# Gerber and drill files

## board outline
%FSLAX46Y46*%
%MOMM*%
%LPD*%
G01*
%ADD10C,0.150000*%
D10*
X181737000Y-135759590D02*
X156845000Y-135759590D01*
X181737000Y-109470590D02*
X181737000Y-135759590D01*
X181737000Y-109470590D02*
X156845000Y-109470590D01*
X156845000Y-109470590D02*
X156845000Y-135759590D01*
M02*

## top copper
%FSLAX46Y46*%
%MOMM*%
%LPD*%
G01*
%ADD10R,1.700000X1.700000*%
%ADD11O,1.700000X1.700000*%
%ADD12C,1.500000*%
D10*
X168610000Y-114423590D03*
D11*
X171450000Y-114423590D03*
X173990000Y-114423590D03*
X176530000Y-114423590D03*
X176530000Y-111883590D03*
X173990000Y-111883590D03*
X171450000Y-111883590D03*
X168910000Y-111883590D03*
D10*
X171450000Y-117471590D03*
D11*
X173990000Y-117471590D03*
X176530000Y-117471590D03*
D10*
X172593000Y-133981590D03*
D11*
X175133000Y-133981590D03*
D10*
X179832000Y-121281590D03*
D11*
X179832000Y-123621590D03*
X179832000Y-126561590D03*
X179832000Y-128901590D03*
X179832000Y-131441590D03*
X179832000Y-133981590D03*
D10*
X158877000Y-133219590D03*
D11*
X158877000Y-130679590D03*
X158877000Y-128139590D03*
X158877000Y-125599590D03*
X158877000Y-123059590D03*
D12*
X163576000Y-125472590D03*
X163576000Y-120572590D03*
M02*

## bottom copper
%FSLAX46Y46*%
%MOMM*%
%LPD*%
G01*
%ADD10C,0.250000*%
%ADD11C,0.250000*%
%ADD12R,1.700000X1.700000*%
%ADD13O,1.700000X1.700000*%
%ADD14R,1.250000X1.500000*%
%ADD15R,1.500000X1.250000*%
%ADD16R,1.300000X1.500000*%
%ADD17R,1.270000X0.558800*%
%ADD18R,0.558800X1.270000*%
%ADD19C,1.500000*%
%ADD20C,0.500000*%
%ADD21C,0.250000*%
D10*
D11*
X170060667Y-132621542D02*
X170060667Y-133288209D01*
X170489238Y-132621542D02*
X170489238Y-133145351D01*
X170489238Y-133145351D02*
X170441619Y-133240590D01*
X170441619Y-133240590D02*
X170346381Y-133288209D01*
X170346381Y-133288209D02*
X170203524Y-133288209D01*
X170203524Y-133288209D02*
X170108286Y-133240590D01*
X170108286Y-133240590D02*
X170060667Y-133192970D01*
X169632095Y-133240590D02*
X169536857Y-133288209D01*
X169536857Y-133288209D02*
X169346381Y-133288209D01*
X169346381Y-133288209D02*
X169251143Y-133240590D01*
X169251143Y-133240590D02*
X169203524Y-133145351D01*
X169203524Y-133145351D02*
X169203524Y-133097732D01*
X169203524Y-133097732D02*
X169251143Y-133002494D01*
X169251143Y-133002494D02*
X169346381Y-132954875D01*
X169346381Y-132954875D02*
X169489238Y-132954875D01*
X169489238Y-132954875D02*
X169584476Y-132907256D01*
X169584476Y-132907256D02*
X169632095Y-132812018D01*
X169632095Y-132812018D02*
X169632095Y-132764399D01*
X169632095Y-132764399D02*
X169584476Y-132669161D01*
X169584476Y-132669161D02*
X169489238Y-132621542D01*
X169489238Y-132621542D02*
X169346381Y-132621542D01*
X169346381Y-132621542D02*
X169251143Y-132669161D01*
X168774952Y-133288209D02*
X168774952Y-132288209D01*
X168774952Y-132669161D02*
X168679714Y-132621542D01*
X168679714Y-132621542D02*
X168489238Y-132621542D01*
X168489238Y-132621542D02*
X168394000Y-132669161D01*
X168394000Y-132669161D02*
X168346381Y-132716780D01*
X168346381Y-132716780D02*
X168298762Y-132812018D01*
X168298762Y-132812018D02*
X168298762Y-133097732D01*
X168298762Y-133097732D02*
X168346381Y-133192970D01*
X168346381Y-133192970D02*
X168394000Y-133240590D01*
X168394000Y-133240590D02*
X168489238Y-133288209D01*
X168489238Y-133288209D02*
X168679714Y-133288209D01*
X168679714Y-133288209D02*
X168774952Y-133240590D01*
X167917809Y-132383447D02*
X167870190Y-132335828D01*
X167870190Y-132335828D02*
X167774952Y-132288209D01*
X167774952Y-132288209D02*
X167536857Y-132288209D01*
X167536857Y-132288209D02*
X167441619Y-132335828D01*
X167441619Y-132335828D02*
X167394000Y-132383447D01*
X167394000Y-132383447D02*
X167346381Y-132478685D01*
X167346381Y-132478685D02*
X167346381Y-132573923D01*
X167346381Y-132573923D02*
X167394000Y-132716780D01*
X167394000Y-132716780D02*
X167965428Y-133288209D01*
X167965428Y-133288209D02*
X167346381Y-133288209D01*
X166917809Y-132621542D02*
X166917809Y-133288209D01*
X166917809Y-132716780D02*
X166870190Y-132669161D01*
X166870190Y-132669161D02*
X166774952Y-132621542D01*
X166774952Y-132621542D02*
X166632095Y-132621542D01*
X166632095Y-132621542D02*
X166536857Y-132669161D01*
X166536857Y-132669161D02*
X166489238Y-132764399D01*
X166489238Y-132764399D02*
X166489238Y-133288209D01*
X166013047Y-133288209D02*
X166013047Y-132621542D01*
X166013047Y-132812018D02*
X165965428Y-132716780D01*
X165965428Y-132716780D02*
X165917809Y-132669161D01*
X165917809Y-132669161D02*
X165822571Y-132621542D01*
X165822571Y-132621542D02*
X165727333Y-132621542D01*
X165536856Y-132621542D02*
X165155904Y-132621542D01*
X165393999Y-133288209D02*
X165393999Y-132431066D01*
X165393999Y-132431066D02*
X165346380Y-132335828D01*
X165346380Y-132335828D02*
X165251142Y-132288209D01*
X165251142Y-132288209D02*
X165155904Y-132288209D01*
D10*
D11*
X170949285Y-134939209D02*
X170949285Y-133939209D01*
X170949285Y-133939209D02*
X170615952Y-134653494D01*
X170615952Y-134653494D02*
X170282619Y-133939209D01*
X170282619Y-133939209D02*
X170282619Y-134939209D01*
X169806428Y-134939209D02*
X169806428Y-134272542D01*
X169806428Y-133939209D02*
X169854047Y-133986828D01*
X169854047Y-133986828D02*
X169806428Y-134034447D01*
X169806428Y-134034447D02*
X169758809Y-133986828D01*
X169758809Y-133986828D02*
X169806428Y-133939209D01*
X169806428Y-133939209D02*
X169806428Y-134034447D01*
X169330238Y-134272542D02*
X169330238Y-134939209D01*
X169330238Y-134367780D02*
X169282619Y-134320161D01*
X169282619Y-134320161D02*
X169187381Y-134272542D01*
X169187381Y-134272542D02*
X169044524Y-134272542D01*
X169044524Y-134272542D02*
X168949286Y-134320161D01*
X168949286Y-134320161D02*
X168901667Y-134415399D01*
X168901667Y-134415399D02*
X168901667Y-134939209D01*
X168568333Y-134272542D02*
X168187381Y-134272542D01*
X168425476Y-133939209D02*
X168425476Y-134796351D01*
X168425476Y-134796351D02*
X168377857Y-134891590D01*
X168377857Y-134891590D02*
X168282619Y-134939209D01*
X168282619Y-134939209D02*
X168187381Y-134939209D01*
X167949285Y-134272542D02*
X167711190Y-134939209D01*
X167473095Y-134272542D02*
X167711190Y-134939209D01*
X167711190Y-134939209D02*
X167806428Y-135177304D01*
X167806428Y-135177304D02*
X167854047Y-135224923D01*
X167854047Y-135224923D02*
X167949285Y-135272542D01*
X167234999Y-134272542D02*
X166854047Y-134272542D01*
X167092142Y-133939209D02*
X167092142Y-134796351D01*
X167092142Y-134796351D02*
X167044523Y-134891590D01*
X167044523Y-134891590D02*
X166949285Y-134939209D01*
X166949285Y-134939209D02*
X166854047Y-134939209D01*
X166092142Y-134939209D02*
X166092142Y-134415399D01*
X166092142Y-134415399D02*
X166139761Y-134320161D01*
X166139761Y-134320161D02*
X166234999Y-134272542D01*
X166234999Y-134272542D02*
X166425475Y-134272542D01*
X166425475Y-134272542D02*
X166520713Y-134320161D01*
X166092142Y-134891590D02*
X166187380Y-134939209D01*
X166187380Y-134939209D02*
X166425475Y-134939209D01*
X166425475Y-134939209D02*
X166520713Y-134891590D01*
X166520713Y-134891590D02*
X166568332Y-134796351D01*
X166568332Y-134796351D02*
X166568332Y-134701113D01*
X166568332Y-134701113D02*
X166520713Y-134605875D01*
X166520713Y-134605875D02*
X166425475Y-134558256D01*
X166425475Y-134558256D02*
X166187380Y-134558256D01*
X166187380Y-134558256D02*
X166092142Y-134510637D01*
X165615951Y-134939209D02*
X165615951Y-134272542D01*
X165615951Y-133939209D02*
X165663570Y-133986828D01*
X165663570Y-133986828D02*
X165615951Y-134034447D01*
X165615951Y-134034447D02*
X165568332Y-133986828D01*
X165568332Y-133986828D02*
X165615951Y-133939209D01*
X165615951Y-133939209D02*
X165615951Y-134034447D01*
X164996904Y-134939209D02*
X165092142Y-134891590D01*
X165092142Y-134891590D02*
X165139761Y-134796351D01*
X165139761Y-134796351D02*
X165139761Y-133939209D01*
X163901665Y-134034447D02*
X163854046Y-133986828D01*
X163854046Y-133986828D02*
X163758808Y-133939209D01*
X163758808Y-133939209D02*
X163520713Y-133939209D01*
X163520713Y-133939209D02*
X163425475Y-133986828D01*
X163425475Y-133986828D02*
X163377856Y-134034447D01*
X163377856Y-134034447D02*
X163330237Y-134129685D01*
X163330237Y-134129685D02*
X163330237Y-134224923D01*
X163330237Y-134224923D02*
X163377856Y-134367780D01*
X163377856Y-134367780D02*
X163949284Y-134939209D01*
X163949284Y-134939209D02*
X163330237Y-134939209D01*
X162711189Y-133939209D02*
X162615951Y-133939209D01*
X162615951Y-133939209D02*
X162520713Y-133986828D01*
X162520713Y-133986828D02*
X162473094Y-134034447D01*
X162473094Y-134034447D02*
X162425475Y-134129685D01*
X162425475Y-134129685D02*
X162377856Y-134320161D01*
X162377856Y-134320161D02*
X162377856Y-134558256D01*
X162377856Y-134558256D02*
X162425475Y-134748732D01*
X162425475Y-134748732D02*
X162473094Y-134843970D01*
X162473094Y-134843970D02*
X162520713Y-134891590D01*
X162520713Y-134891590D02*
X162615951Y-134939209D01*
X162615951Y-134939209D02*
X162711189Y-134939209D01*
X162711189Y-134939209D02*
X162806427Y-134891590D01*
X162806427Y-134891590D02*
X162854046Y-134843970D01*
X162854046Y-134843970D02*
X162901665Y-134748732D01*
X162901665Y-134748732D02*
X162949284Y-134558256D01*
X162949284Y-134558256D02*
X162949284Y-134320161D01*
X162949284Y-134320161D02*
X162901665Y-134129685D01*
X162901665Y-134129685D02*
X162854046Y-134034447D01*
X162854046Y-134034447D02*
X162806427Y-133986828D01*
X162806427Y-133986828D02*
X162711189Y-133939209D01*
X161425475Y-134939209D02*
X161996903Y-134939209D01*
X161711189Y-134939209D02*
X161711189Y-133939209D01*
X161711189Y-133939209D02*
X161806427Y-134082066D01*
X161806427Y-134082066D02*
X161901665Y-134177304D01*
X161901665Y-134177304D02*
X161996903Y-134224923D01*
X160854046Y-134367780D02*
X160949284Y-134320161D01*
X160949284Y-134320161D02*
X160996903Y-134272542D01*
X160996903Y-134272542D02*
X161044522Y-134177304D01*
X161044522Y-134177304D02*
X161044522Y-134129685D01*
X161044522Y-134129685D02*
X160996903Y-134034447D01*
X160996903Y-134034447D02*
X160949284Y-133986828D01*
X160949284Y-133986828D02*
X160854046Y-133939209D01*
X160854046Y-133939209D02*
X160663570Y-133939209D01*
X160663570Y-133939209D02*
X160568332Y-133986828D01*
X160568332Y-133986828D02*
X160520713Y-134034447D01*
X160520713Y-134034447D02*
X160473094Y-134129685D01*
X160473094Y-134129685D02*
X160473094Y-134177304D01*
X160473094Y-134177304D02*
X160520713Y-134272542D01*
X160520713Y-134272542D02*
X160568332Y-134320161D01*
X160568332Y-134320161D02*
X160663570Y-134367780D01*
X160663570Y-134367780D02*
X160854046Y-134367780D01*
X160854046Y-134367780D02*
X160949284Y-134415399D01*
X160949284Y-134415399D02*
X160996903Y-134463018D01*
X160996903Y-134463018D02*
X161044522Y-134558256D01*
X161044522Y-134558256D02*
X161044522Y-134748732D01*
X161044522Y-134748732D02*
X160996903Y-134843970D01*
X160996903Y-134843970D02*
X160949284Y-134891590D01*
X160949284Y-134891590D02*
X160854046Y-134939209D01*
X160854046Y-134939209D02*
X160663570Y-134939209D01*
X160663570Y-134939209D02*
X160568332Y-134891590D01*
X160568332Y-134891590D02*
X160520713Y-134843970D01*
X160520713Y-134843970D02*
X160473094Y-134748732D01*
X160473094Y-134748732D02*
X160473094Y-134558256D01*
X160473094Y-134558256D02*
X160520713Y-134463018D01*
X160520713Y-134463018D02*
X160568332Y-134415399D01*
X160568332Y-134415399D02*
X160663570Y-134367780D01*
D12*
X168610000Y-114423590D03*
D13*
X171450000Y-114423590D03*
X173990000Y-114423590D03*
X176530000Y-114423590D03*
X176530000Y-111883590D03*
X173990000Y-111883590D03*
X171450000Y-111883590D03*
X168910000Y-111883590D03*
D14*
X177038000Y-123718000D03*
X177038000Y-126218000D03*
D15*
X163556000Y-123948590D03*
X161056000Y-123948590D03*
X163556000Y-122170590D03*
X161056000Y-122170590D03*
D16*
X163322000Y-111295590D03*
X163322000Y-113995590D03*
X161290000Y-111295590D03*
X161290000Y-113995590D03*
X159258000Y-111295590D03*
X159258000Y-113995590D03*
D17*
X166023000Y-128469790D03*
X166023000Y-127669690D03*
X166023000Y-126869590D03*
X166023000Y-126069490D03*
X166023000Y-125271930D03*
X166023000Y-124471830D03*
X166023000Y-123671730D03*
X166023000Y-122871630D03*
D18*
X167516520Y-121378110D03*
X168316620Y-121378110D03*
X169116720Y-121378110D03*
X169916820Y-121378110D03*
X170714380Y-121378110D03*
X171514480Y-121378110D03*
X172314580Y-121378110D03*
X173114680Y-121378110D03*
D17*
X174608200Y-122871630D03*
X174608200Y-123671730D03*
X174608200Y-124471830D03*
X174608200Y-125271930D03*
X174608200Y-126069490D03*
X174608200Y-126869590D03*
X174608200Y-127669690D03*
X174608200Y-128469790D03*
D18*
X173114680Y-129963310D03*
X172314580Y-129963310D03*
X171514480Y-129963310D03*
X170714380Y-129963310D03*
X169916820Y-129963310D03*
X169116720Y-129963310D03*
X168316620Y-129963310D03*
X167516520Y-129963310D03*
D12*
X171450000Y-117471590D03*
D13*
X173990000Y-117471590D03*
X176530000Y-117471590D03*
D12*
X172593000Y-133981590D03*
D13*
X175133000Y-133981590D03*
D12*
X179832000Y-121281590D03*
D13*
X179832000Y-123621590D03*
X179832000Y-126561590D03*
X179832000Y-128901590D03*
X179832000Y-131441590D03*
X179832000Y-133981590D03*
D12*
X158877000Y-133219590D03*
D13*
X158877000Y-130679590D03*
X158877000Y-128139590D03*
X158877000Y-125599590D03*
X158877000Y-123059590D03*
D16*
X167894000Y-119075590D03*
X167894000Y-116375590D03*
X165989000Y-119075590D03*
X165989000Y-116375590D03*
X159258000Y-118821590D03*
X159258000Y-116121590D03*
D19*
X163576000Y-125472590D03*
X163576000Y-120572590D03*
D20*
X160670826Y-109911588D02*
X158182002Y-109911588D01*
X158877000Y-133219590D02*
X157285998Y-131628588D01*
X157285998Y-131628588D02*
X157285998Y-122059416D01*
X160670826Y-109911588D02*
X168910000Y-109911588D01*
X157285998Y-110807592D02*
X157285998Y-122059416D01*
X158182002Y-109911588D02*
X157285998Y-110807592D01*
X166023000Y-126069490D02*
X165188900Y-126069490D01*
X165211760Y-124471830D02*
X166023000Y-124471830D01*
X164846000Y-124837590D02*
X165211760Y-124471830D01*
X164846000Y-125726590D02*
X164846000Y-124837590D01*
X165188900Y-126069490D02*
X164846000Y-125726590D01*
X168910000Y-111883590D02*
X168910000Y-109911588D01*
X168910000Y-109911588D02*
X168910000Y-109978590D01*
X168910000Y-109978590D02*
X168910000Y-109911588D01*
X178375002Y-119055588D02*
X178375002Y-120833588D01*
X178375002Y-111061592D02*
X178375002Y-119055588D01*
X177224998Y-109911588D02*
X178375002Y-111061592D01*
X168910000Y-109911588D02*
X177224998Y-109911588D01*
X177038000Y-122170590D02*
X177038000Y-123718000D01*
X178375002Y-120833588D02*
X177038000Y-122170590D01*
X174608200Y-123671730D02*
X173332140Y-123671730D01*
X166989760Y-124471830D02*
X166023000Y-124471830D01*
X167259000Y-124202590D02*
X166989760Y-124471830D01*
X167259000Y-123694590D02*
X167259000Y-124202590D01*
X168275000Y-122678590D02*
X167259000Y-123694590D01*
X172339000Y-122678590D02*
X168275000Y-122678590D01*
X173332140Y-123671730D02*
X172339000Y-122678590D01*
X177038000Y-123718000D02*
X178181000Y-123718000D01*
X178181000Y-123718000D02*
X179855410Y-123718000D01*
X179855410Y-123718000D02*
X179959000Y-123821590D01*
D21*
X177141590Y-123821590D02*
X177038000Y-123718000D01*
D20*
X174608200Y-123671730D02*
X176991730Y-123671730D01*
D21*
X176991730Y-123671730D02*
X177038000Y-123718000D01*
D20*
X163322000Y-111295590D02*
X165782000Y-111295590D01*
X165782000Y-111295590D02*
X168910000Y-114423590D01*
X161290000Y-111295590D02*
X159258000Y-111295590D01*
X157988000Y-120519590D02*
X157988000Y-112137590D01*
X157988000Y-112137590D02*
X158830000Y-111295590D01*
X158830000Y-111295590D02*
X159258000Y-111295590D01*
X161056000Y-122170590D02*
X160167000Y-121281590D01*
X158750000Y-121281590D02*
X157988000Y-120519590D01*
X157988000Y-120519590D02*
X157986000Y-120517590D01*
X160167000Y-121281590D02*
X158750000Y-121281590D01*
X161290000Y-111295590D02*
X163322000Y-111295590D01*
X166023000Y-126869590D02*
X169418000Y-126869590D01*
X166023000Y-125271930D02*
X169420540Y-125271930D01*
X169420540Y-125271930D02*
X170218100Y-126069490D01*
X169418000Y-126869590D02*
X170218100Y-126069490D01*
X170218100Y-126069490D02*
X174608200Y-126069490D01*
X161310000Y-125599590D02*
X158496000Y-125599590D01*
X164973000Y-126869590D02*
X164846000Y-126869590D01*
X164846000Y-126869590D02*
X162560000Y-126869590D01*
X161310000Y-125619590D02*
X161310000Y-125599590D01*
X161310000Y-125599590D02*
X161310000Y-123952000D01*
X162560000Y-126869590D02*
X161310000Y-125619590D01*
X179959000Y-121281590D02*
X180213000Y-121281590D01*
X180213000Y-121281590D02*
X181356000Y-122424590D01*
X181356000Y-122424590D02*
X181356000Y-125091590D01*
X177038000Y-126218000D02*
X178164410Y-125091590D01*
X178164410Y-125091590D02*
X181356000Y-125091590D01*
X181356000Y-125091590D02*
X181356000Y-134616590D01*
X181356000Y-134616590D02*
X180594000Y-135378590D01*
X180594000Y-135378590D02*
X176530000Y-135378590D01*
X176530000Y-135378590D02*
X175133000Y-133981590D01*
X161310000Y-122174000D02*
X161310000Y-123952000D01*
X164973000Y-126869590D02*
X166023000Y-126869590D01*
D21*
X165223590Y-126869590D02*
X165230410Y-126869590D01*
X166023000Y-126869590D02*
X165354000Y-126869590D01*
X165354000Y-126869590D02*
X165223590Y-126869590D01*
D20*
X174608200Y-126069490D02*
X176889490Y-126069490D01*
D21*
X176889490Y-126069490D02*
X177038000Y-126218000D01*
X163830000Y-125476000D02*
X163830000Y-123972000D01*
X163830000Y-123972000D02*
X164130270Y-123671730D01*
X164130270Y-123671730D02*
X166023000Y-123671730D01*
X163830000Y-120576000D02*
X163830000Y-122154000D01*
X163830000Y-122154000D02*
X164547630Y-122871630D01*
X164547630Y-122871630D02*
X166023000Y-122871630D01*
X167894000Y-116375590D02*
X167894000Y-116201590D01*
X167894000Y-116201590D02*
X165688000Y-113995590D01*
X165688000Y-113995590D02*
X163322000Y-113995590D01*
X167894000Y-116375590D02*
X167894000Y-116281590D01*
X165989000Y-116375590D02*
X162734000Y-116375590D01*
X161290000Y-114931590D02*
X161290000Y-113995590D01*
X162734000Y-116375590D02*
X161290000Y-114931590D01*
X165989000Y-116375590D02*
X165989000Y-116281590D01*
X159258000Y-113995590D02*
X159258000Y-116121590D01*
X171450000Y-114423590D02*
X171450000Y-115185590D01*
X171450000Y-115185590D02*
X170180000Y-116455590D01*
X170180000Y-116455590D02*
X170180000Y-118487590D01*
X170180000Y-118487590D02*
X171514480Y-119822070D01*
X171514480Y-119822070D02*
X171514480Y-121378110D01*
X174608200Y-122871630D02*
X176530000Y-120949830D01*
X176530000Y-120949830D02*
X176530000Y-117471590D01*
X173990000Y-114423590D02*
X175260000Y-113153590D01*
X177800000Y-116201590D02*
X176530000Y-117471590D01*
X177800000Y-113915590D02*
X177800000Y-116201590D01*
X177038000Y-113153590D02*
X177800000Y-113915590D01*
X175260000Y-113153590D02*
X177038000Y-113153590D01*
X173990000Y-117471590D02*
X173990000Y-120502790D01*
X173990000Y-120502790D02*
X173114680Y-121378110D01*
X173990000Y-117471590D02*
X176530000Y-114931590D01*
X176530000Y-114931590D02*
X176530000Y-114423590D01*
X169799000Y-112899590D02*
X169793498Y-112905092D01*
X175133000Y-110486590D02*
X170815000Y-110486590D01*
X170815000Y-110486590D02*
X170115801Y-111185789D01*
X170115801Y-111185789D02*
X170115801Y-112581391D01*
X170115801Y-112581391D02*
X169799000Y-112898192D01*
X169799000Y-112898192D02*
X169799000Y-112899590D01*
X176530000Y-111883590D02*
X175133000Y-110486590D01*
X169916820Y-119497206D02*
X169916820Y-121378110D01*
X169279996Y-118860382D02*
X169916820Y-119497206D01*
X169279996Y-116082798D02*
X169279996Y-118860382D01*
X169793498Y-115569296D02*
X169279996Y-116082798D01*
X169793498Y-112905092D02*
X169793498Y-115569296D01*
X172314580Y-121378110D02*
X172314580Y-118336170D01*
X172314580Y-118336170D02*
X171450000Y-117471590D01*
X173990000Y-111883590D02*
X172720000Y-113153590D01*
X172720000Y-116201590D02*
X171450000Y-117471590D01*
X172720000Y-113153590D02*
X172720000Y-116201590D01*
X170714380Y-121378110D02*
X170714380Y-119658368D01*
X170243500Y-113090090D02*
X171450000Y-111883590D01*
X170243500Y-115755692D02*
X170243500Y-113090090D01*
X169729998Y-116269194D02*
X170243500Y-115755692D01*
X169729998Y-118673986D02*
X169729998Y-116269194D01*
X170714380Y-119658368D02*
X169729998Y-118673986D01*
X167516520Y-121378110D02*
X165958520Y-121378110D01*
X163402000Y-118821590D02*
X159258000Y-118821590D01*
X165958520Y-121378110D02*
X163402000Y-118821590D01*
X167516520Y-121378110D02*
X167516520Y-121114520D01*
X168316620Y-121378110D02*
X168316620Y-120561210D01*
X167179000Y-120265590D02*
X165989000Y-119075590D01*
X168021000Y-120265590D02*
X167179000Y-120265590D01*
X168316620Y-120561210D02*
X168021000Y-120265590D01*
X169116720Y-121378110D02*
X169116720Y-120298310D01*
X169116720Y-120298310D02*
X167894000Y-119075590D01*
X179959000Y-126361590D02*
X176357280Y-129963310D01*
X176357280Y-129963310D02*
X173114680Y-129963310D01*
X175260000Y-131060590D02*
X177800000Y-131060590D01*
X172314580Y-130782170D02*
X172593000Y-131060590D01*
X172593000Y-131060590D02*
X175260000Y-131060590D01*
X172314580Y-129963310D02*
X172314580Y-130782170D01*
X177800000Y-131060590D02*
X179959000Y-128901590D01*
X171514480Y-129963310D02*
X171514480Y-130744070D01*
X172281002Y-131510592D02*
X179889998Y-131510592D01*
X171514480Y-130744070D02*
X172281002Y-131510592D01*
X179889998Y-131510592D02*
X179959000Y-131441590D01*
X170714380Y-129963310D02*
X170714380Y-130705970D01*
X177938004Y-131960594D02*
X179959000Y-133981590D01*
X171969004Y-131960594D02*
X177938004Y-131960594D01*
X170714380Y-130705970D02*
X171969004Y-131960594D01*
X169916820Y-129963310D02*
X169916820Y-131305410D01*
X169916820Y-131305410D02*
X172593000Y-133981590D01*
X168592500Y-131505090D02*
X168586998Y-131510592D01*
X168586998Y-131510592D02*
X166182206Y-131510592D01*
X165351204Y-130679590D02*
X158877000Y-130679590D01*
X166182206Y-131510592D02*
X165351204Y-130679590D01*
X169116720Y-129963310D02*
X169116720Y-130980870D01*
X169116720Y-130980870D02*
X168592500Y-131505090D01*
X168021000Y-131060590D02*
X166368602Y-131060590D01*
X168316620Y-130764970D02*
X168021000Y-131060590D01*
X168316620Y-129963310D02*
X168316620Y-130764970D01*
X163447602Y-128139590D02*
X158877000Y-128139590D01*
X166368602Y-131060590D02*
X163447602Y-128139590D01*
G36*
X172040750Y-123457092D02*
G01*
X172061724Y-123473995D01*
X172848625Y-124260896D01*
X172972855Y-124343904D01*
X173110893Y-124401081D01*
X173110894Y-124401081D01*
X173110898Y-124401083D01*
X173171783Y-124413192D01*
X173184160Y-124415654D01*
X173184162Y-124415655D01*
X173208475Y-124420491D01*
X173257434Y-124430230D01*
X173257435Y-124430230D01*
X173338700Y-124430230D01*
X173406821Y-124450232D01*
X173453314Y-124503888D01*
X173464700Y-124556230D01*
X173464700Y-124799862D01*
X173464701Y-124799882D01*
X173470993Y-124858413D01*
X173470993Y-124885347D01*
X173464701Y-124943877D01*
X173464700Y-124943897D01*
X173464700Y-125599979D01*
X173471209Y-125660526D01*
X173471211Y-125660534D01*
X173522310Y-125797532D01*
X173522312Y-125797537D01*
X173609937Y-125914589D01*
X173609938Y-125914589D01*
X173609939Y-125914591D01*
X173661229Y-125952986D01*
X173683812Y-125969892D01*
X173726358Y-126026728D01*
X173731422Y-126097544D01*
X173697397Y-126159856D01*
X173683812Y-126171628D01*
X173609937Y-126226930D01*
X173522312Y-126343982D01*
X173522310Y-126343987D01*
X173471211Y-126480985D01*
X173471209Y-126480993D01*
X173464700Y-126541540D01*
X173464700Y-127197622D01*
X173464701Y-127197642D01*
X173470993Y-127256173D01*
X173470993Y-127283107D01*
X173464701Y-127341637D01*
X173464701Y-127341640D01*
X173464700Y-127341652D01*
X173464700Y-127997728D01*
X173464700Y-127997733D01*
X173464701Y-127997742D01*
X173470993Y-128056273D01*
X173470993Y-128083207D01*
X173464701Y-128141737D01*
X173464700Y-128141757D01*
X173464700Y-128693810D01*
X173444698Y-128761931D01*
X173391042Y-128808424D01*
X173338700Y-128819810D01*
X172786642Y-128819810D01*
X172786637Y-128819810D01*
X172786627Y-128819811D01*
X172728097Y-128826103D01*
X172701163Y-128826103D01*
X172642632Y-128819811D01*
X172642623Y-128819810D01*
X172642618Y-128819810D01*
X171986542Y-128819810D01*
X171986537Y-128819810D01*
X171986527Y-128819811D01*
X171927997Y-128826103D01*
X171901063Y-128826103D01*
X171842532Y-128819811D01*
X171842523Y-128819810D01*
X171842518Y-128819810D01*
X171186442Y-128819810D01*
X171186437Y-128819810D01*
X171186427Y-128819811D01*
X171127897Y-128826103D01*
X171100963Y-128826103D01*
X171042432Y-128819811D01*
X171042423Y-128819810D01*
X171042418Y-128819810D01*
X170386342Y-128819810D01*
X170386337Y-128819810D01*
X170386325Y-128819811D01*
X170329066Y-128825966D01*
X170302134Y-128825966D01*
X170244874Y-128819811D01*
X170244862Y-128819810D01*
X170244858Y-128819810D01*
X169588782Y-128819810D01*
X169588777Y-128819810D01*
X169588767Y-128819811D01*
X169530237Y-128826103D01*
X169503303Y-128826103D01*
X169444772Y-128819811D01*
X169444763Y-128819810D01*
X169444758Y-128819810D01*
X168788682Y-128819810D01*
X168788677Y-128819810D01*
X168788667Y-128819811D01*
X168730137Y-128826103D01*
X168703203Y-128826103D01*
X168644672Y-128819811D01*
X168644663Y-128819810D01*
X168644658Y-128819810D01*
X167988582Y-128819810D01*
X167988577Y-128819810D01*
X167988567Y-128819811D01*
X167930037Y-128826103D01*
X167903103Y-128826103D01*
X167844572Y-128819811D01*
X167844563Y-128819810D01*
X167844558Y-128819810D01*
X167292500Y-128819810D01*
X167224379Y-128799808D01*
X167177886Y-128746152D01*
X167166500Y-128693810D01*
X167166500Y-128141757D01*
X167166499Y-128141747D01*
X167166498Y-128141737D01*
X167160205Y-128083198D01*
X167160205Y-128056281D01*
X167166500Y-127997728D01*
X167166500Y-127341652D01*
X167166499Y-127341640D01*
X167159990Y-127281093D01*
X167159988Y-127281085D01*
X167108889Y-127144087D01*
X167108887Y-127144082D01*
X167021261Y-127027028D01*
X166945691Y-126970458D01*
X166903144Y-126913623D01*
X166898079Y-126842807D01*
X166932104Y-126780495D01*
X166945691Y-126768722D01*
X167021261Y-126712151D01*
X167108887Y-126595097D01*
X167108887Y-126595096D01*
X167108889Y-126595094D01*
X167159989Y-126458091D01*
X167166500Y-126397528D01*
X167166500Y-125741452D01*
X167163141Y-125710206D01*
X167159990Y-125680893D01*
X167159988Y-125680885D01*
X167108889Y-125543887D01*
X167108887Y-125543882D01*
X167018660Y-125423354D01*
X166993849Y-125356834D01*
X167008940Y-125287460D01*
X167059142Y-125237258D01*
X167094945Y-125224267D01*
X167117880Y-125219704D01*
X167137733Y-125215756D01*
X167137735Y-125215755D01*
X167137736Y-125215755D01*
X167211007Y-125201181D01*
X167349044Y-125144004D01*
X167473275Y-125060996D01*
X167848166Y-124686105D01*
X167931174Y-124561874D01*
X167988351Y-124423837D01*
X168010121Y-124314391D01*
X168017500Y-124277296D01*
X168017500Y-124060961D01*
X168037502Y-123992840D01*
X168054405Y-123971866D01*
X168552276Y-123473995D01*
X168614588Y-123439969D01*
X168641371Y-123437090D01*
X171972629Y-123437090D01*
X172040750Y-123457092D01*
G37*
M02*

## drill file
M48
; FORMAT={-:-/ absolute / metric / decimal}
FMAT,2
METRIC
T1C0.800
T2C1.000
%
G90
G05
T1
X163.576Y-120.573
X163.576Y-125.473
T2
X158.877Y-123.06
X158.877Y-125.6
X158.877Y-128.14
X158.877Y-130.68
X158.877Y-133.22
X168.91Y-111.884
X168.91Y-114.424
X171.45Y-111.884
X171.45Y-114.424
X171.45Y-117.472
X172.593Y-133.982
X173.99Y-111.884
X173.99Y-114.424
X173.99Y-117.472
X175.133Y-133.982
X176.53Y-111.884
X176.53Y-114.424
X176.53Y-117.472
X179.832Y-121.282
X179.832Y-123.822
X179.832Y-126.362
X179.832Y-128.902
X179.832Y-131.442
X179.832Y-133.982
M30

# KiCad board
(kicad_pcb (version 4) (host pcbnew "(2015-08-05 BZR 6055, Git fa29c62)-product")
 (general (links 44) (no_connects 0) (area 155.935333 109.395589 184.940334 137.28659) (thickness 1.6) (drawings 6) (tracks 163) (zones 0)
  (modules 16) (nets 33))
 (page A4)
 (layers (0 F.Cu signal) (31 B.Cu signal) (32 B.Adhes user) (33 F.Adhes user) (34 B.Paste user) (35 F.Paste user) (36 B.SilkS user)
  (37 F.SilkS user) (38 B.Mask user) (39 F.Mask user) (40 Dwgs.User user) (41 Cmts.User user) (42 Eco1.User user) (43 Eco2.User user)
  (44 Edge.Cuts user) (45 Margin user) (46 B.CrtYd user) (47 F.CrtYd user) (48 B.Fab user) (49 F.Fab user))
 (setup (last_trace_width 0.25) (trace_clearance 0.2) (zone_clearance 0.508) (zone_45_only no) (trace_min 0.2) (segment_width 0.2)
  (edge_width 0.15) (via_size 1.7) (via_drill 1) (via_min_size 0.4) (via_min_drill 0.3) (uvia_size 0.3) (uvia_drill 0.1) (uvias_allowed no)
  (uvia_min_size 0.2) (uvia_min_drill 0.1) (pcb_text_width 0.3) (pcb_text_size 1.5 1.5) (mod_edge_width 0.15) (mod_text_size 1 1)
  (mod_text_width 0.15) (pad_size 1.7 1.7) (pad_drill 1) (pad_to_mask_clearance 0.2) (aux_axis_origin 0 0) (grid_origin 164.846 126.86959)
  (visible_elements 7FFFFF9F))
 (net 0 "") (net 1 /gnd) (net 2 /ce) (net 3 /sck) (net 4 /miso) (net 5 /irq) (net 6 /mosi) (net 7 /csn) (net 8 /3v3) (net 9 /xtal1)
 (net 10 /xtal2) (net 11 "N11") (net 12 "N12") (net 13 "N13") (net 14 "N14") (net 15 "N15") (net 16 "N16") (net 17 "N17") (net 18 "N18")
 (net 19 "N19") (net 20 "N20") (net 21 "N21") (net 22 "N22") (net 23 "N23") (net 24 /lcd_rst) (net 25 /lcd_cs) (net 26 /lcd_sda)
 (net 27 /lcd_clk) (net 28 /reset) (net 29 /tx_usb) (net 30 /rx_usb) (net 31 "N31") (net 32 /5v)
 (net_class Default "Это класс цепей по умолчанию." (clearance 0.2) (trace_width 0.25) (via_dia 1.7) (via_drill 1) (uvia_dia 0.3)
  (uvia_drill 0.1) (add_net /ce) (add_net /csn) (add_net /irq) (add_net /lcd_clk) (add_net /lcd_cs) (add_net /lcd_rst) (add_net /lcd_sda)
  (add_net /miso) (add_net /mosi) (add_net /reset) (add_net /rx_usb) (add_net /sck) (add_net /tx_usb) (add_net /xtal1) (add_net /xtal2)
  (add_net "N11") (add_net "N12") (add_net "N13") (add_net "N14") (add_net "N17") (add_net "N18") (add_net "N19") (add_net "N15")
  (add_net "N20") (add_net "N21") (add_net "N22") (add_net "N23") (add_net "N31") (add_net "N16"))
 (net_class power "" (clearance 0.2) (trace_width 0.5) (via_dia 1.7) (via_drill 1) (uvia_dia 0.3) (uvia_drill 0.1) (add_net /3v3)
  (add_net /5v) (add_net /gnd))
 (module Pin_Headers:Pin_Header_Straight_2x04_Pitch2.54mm (layer F.Cu) (at 168.91 114.42359 90)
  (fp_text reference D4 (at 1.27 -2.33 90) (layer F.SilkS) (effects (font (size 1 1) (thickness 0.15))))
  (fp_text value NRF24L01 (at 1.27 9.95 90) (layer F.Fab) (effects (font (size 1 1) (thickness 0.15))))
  (pad 1 thru_hole rect (at 0 0 90) (size 1.7 1.7) (drill 1 (offset 0 -0.3)) (layers *.Cu *.Mask) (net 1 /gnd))
  (pad 2 thru_hole oval (at 0 2.54 90) (size 1.7 1.7) (drill 1) (layers *.Cu *.Mask) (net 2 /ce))
  (pad 3 thru_hole oval (at 0 5.08 90) (size 1.7 1.7) (drill 1) (layers *.Cu *.Mask) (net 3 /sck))
  (pad 4 thru_hole oval (at 0 7.62 90) (size 1.7 1.7) (drill 1) (layers *.Cu *.Mask) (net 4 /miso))
  (pad 5 thru_hole oval (at 2.54 7.62 90) (size 1.7 1.7) (drill 1) (layers *.Cu *.Mask) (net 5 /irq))
  (pad 6 thru_hole oval (at 2.54 5.08 90) (size 1.7 1.7) (drill 1) (layers *.Cu *.Mask) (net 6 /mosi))
  (pad 7 thru_hole oval (at 2.54 2.54 90) (size 1.7 1.7) (drill 1) (layers *.Cu *.Mask) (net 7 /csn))
  (pad 8 thru_hole oval (at 2.54 0 90) (size 1.7 1.7) (drill 1) (layers *.Cu *.Mask) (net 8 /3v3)))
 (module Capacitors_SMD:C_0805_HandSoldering (layer B.Cu) (at 177.038 124.968 270)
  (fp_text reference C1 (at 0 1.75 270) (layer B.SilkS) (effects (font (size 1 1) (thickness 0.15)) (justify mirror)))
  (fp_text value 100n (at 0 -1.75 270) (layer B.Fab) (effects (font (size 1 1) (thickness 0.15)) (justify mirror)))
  (pad 1 smd rect (at -1.25 0 270) (size 1.5 1.25) (layers B.Cu B.Paste B.Mask) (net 8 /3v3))
  (pad 2 smd rect (at 1.25 0 270) (size 1.5 1.25) (layers B.Cu B.Paste B.Mask) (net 1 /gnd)))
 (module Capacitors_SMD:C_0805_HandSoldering (layer B.Cu) (at 162.306 123.94859 180)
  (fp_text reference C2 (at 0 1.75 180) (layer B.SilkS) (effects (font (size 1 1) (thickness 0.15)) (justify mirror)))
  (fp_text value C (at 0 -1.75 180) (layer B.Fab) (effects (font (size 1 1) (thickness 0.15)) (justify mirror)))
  (pad 1 smd rect (at -1.25 0 180) (size 1.5 1.25) (layers B.Cu B.Paste B.Mask) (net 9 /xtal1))
  (pad 2 smd rect (at 1.25 0 180) (size 1.5 1.25) (layers B.Cu B.Paste B.Mask) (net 1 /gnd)))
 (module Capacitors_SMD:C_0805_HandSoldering (layer B.Cu) (at 162.306 122.17059 180)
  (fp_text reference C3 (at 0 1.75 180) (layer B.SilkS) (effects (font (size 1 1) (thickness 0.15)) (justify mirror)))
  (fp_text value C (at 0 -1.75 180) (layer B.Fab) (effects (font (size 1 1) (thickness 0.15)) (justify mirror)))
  (pad 1 smd rect (at -1.25 0 180) (size 1.5 1.25) (layers B.Cu B.Paste B.Mask) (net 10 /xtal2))
  (pad 2 smd rect (at 1.25 0 180) (size 1.5 1.25) (layers B.Cu B.Paste B.Mask) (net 1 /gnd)))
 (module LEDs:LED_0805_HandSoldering (layer B.Cu) (at 163.322 112.64559 270)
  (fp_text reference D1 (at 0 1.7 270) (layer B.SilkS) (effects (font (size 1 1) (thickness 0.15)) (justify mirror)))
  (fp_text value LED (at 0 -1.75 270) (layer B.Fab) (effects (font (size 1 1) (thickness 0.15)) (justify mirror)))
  (pad 1 smd rect (at -1.35 0 270) (size 1.5 1.3) (layers B.Cu B.Paste B.Mask) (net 1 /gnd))
  (pad 2 smd rect (at 1.35 0 270) (size 1.5 1.3) (layers B.Cu B.Paste B.Mask) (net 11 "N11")))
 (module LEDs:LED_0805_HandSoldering (layer B.Cu) (at 161.29 112.64559 270)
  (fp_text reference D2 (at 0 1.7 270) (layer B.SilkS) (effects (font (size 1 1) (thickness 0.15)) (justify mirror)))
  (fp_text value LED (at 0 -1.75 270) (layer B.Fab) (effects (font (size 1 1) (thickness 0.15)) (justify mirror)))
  (pad 1 smd rect (at -1.35 0 270) (size 1.5 1.3) (layers B.Cu B.Paste B.Mask) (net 1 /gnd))
  (pad 2 smd rect (at 1.35 0 270) (size 1.5 1.3) (layers B.Cu B.Paste B.Mask) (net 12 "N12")))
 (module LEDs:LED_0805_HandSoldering (layer B.Cu) (at 159.258 112.64559 270)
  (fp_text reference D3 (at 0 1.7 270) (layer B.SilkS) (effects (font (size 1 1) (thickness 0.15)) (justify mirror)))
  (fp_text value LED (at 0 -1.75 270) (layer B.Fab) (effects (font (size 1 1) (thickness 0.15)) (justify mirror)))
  (pad 1 smd rect (at -1.35 0 270) (size 1.5 1.3) (layers B.Cu B.Paste B.Mask) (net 1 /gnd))
  (pad 2 smd rect (at 1.35 0 270) (size 1.5 1.3) (layers B.Cu B.Paste B.Mask) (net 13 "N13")))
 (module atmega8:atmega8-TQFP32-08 (layer B.Cu) (at 170.3156 125.67071)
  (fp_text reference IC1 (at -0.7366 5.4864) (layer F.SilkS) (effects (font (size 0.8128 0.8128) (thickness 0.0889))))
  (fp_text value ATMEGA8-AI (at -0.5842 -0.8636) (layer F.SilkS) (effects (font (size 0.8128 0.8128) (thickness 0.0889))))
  (pad 1 smd rect (at -4.2926 2.79908) (size 1.27 0.5588) (layers B.Cu B.Paste B.Mask) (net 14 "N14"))
  (pad 2 smd rect (at -4.2926 1.99898) (size 1.27 0.5588) (layers B.Cu B.Paste B.Mask) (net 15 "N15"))
  (pad 3 smd rect (at -4.2926 1.19888) (size 1.27 0.5588) (layers B.Cu B.Paste B.Mask) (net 1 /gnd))
  (pad 4 smd rect (at -4.2926 0.39878) (size 1.27 0.5588) (layers B.Cu B.Paste B.Mask) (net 8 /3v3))
  (pad 5 smd rect (at -4.2926 -0.39878) (size 1.27 0.5588) (layers B.Cu B.Paste B.Mask) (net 1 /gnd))
  (pad 6 smd rect (at -4.2926 -1.19888) (size 1.27 0.5588) (layers B.Cu B.Paste B.Mask) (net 8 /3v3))
  (pad 7 smd rect (at -4.2926 -1.99898) (size 1.27 0.5588) (layers B.Cu B.Paste B.Mask) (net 9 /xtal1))
  (pad 8 smd rect (at -4.2926 -2.79908) (size 1.27 0.5588) (layers B.Cu B.Paste B.Mask) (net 10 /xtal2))
  (pad 9 smd rect (at -2.79908 -4.2926) (size 0.5588 1.27) (layers B.Cu B.Paste B.Mask) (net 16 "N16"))
  (pad 10 smd rect (at -1.99898 -4.2926) (size 0.5588 1.27) (layers B.Cu B.Paste B.Mask) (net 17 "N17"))
  (pad 11 smd rect (at -1.19888 -4.2926) (size 0.5588 1.27) (layers B.Cu B.Paste B.Mask) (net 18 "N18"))
  (pad 12 smd rect (at -0.39878 -4.2926) (size 0.5588 1.27) (layers B.Cu B.Paste B.Mask) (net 5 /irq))
  (pad 13 smd rect (at 0.39878 -4.2926) (size 0.5588 1.27) (layers B.Cu B.Paste B.Mask) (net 7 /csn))
  (pad 14 smd rect (at 1.19888 -4.2926) (size 0.5588 1.27) (layers B.Cu B.Paste B.Mask) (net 2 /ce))
  (pad 15 smd rect (at 1.99898 -4.2926) (size 0.5588 1.27) (layers B.Cu B.Paste B.Mask) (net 6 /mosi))
  (pad 16 smd rect (at 2.79908 -4.2926) (size 0.5588 1.27) (layers B.Cu B.Paste B.Mask) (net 4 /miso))
  (pad 17 smd rect (at 4.2926 -2.79908) (size 1.27 0.5588) (layers B.Cu B.Paste B.Mask) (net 3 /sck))
  (pad 18 smd rect (at 4.2926 -1.99898) (size 1.27 0.5588) (layers B.Cu B.Paste B.Mask) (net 8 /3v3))
  (pad 19 smd rect (at 4.2926 -1.19888) (size 1.27 0.5588) (layers B.Cu B.Paste B.Mask) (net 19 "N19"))
  (pad 20 smd rect (at 4.2926 -0.39878) (size 1.27 0.5588) (layers B.Cu B.Paste B.Mask) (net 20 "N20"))
  (pad 21 smd rect (at 4.2926 0.39878) (size 1.27 0.5588) (layers B.Cu B.Paste B.Mask) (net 1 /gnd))
  (pad 22 smd rect (at 4.2926 1.19888) (size 1.27 0.5588) (layers B.Cu B.Paste B.Mask) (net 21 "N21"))
  (pad 23 smd rect (at 4.2926 1.99898) (size 1.27 0.5588) (layers B.Cu B.Paste B.Mask) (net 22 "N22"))
  (pad 24 smd rect (at 4.2926 2.79908) (size 1.27 0.5588) (layers B.Cu B.Paste B.Mask) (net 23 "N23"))
  (pad 25 smd rect (at 2.79908 4.2926) (size 0.5588 1.27) (layers B.Cu B.Paste B.Mask) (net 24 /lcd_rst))
  (pad 26 smd rect (at 1.99898 4.2926) (size 0.5588 1.27) (layers B.Cu B.Paste B.Mask) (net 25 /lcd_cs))
  (pad 27 smd rect (at 1.19888 4.2926) (size 0.5588 1.27) (layers B.Cu B.Paste B.Mask) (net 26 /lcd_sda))
  (pad 28 smd rect (at 0.39878 4.2926) (size 0.5588 1.27) (layers B.Cu B.Paste B.Mask) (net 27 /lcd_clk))
  (pad 29 smd rect (at -0.39878 4.2926) (size 0.5588 1.27) (layers B.Cu B.Paste B.Mask) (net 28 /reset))
  (pad 30 smd rect (at -1.19888 4.2926) (size 0.5588 1.27) (layers B.Cu B.Paste B.Mask) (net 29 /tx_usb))
  (pad 31 smd rect (at -1.99898 4.2926) (size 0.5588 1.27) (layers B.Cu B.Paste B.Mask) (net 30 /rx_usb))
  (pad 32 smd rect (at -2.79908 4.2926) (size 0.5588 1.27) (layers B.Cu B.Paste B.Mask) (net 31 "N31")))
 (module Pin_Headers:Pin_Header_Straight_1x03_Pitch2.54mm (layer F.Cu) (at 171.45 117.47159 90)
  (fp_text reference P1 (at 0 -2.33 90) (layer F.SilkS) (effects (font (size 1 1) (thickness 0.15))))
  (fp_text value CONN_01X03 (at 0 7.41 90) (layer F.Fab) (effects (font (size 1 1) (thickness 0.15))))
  (pad 1 thru_hole rect (at 0 0 90) (size 1.7 1.7) (drill 1) (layers *.Cu *.Mask) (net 6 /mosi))
  (pad 2 thru_hole oval (at 0 2.54 90) (size 1.7 1.7) (drill 1) (layers *.Cu *.Mask) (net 4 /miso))
  (pad 3 thru_hole oval (at 0 5.08 90) (size 1.7 1.7) (drill 1) (layers *.Cu *.Mask) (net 3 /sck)))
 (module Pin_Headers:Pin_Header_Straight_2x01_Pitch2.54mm (layer F.Cu) (at 172.593 133.98159)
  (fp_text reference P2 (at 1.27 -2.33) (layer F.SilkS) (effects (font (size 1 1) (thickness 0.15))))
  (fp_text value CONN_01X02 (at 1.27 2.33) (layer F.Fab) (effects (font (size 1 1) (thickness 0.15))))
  (pad 1 thru_hole rect (at 0 0) (size 1.7 1.7) (drill 1) (layers *.Cu *.Mask) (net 28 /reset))
  (pad 2 thru_hole oval (at 2.54 0) (size 1.7 1.7) (drill 1) (layers *.Cu *.Mask) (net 1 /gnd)))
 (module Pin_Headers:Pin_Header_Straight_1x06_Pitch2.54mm (layer F.Cu) (at 179.832 121.28159)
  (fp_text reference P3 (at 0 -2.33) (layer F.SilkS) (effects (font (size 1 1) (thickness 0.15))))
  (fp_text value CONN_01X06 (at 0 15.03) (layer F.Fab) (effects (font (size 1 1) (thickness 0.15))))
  (pad 1 thru_hole rect (at 0 0) (size 1.7 1.7) (drill 1) (layers *.Cu *.Mask) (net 1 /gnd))
  (pad 2 thru_hole oval (at 0 2.54) (size 1.7 1.7) (drill 1 (offset 0 -0.2)) (layers *.Cu *.Mask) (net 8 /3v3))
  (pad 3 thru_hole oval (at 0 5.08) (size 1.7 1.7) (drill 1 (offset 0 0.2)) (layers *.Cu *.Mask) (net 24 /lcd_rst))
  (pad 4 thru_hole oval (at 0 7.62) (size 1.7 1.7) (drill 1) (layers *.Cu *.Mask) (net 25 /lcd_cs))
  (pad 5 thru_hole oval (at 0 10.16) (size 1.7 1.7) (drill 1) (layers *.Cu *.Mask) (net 26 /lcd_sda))
  (pad 6 thru_hole oval (at 0 12.7) (size 1.7 1.7) (drill 1) (layers *.Cu *.Mask) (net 27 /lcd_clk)))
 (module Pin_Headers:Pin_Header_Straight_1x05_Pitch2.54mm (layer F.Cu) (at 158.877 133.21959 180)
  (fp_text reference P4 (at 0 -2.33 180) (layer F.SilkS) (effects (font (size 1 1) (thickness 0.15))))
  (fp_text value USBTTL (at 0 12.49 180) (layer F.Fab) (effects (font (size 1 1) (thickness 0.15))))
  (pad 1 thru_hole rect (at 0 0 180) (size 1.7 1.7) (drill 1) (layers *.Cu *.Mask) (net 8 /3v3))
  (pad 2 thru_hole oval (at 0 2.54 180) (size 1.7 1.7) (drill 1) (layers *.Cu *.Mask) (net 29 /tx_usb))
  (pad 3 thru_hole oval (at 0 5.08 180) (size 1.7 1.7) (drill 1) (layers *.Cu *.Mask) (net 30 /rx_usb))
  (pad 4 thru_hole oval (at 0 7.62 180) (size 1.7 1.7) (drill 1) (layers *.Cu *.Mask) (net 1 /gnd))
  (pad 5 thru_hole oval (at 0 10.16 180) (size 1.7 1.7) (drill 1) (layers *.Cu *.Mask) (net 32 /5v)))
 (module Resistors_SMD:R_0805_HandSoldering (layer B.Cu) (at 167.894 117.72559 90)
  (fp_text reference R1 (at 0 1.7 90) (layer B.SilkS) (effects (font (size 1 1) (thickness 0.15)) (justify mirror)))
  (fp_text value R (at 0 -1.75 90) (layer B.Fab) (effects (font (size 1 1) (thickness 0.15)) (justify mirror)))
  (pad 1 smd rect (at -1.35 0 90) (size 1.5 1.3) (layers B.Cu B.Paste B.Mask) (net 18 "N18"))
  (pad 2 smd rect (at 1.35 0 90) (size 1.5 1.3) (layers B.Cu B.Paste B.Mask) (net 11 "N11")))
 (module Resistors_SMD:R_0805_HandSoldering (layer B.Cu) (at 165.989 117.72559 90)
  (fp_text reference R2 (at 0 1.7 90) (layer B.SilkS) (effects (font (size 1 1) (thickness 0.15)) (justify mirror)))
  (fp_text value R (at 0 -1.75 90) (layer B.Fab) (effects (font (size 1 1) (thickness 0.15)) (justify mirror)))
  (pad 1 smd rect (at -1.35 0 90) (size 1.5 1.3) (layers B.Cu B.Paste B.Mask) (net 17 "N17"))
  (pad 2 smd rect (at 1.35 0 90) (size 1.5 1.3) (layers B.Cu B.Paste B.Mask) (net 12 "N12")))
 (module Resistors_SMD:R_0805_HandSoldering (layer B.Cu) (at 159.258 117.47159 90)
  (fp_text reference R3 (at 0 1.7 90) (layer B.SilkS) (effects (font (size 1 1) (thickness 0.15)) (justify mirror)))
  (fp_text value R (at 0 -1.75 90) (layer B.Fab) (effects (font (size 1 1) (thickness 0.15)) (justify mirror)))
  (pad 1 smd rect (at -1.35 0 90) (size 1.5 1.3) (layers B.Cu B.Paste B.Mask) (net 16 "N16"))
  (pad 2 smd rect (at 1.35 0 90) (size 1.5 1.3) (layers B.Cu B.Paste B.Mask) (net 13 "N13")))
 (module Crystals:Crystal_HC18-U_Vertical (layer F.Cu) (at 163.576 125.47259 90)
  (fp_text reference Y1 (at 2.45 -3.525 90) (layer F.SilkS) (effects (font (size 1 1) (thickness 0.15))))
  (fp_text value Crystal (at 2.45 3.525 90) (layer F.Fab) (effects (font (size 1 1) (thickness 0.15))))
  (pad 1 thru_hole circle (at 0 0 90) (size 1.5 1.5) (drill 0.8) (layers *.Cu *.Mask) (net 9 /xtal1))
  (pad 2 thru_hole circle (at 4.9 0 90) (size 1.5 1.5) (drill 0.8) (layers *.Cu *.Mask) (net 10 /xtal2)))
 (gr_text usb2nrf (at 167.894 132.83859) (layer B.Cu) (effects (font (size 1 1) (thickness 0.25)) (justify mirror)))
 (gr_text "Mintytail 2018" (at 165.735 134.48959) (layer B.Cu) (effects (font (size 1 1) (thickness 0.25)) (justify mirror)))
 (gr_line (start 181.737 135.75959) (end 156.845 135.75959) (angle 90) (layer Edge.Cuts) (width 0.15))
 (gr_line (start 181.737 109.47059) (end 181.737 135.75959) (angle 90) (layer Edge.Cuts) (width 0.15))
 (gr_line (start 181.737 109.47059) (end 156.845 109.47059) (angle 90) (layer Edge.Cuts) (width 0.15))
 (gr_line (start 156.845 109.47059) (end 156.845 135.75959) (angle 90) (layer Edge.Cuts) (width 0.15))
 (segment (start 160.670826 109.911588) (end 158.182002 109.911588) (width 0.5) (layer B.Cu) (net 8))
 (segment (start 158.877 133.21959) (end 157.285998 131.628588) (width 0.5) (layer B.Cu) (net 8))
 (segment (start 157.285998 131.628588) (end 157.285998 122.059416) (width 0.5) (layer B.Cu) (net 8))
 (segment (start 160.670826 109.911588) (end 168.91 109.911588) (width 0.5) (layer B.Cu) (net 8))
 (segment (start 157.285998 110.807592) (end 157.285998 122.059416) (width 0.5) (layer B.Cu) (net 8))
 (segment (start 158.182002 109.911588) (end 157.285998 110.807592) (width 0.5) (layer B.Cu) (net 8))
 (segment (start 166.023 126.06949) (end 165.1889 126.06949) (width 0.5) (layer B.Cu) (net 8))
 (segment (start 165.21176 124.47183) (end 166.023 124.47183) (width 0.5) (layer B.Cu) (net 8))
 (segment (start 164.846 124.83759) (end 165.21176 124.47183) (width 0.5) (layer B.Cu) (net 8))
 (segment (start 164.846 125.72659) (end 164.846 124.83759) (width 0.5) (layer B.Cu) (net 8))
 (segment (start 165.1889 126.06949) (end 164.846 125.72659) (width 0.5) (layer B.Cu) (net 8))
 (segment (start 168.91 111.88359) (end 168.91 109.911588) (width 0.5) (layer B.Cu) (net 8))
 (segment (start 168.91 109.911588) (end 168.91 109.97859) (width 0.5) (layer B.Cu) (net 8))
 (segment (start 168.91 109.97859) (end 168.91 109.911588) (width 0.5) (layer B.Cu) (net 8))
 (segment (start 178.375002 119.055588) (end 178.375002 120.833588) (width 0.5) (layer B.Cu) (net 8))
 (segment (start 178.375002 111.061592) (end 178.375002 119.055588) (width 0.5) (layer B.Cu) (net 8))
 (segment (start 177.224998 109.911588) (end 178.375002 111.061592) (width 0.5) (layer B.Cu) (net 8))
 (segment (start 168.91 109.911588) (end 177.224998 109.911588) (width 0.5) (layer B.Cu) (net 8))
 (segment (start 177.038 122.17059) (end 177.038 123.718) (width 0.5) (layer B.Cu) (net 8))
 (segment (start 178.375002 120.833588) (end 177.038 122.17059) (width 0.5) (layer B.Cu) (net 8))
 (segment (start 174.6082 123.67173) (end 173.33214 123.67173) (width 0.5) (layer B.Cu) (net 8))
 (segment (start 166.98976 124.47183) (end 166.023 124.47183) (width 0.5) (layer B.Cu) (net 8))
 (segment (start 167.259 124.20259) (end 166.98976 124.47183) (width 0.5) (layer B.Cu) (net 8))
 (segment (start 167.259 123.69459) (end 167.259 124.20259) (width 0.5) (layer B.Cu) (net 8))
 (segment (start 168.275 122.67859) (end 167.259 123.69459) (width 0.5) (layer B.Cu) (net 8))
 (segment (start 172.339 122.67859) (end 168.275 122.67859) (width 0.5) (layer B.Cu) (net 8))
 (segment (start 173.33214 123.67173) (end 172.339 122.67859) (width 0.5) (layer B.Cu) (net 8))
 (segment (start 177.038 123.718) (end 178.181 123.718) (width 0.5) (layer B.Cu) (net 8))
 (segment (start 178.181 123.718) (end 179.85541 123.718) (width 0.5) (layer B.Cu) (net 8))
 (segment (start 179.85541 123.718) (end 179.959 123.82159) (width 0.5) (layer B.Cu) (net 8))
 (segment (start 177.14159 123.82159) (end 177.038 123.718) (width 0.25) (layer B.Cu) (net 8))
 (segment (start 174.6082 123.67173) (end 176.99173 123.67173) (width 0.5) (layer B.Cu) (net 8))
 (segment (start 176.99173 123.67173) (end 177.038 123.718) (width 0.25) (layer B.Cu) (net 8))
 (segment (start 163.322 111.29559) (end 165.782 111.29559) (width 0.5) (layer B.Cu) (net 1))
 (segment (start 165.782 111.29559) (end 168.91 114.42359) (width 0.5) (layer B.Cu) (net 1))
 (segment (start 161.29 111.29559) (end 159.258 111.29559) (width 0.5) (layer B.Cu) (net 1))
 (segment (start 157.988 120.51959) (end 157.988 112.13759) (width 0.5) (layer B.Cu) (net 1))
 (segment (start 157.988 112.13759) (end 158.83 111.29559) (width 0.5) (layer B.Cu) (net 1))
 (segment (start 158.83 111.29559) (end 159.258 111.29559) (width 0.5) (layer B.Cu) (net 1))
 (segment (start 161.056 122.17059) (end 160.167 121.28159) (width 0.5) (layer B.Cu) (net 1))
 (segment (start 158.75 121.28159) (end 157.988 120.51959) (width 0.5) (layer B.Cu) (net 1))
 (segment (start 157.988 120.51959) (end 157.986 120.51759) (width 0.5) (layer B.Cu) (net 1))
 (segment (start 160.167 121.28159) (end 158.75 121.28159) (width 0.5) (layer B.Cu) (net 1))
 (segment (start 161.29 111.29559) (end 163.322 111.29559) (width 0.5) (layer B.Cu) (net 1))
 (segment (start 166.023 126.86959) (end 169.418 126.86959) (width 0.5) (layer B.Cu) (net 1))
 (segment (start 166.023 125.27193) (end 169.42054 125.27193) (width 0.5) (layer B.Cu) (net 1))
 (segment (start 169.42054 125.27193) (end 170.2181 126.06949) (width 0.5) (layer B.Cu) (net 1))
 (segment (start 169.418 126.86959) (end 170.2181 126.06949) (width 0.5) (layer B.Cu) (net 1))
 (segment (start 170.2181 126.06949) (end 174.6082 126.06949) (width 0.5) (layer B.Cu) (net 1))
 (segment (start 161.31 125.59959) (end 158.496 125.59959) (width 0.5) (layer B.Cu) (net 1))
 (segment (start 164.973 126.86959) (end 164.846 126.86959) (width 0.5) (layer B.Cu) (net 1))
 (segment (start 164.846 126.86959) (end 162.56 126.86959) (width 0.5) (layer B.Cu) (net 1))
 (segment (start 161.31 125.61959) (end 161.31 125.59959) (width 0.5) (layer B.Cu) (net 1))
 (segment (start 161.31 125.59959) (end 161.31 123.952) (width 0.5) (layer B.Cu) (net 1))
 (segment (start 162.56 126.86959) (end 161.31 125.61959) (width 0.5) (layer B.Cu) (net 1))
 (segment (start 179.959 121.28159) (end 180.213 121.28159) (width 0.5) (layer B.Cu) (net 1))
 (segment (start 180.213 121.28159) (end 181.356 122.42459) (width 0.5) (layer B.Cu) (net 1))
 (segment (start 181.356 122.42459) (end 181.356 125.09159) (width 0.5) (layer B.Cu) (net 1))
 (segment (start 177.038 126.218) (end 178.16441 125.09159) (width 0.5) (layer B.Cu) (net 1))
 (segment (start 178.16441 125.09159) (end 181.356 125.09159) (width 0.5) (layer B.Cu) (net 1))
 (segment (start 181.356 125.09159) (end 181.356 134.61659) (width 0.5) (layer B.Cu) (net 1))
 (segment (start 181.356 134.61659) (end 180.594 135.37859) (width 0.5) (layer B.Cu) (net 1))
 (segment (start 180.594 135.37859) (end 176.53 135.37859) (width 0.5) (layer B.Cu) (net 1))
 (segment (start 176.53 135.37859) (end 175.133 133.98159) (width 0.5) (layer B.Cu) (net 1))
 (segment (start 161.31 122.174) (end 161.31 123.952) (width 0.5) (layer B.Cu) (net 1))
 (segment (start 164.973 126.86959) (end 166.023 126.86959) (width 0.5) (layer B.Cu) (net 1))
 (segment (start 165.22359 126.86959) (end 165.23041 126.86959) (width 0.25) (layer B.Cu) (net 1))
 (segment (start 166.023 126.86959) (end 165.354 126.86959) (width 0.25) (layer B.Cu) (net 1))
 (segment (start 165.354 126.86959) (end 165.22359 126.86959) (width 0.25) (layer B.Cu) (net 1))
 (segment (start 174.6082 126.06949) (end 176.88949 126.06949) (width 0.5) (layer B.Cu) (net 1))
 (segment (start 176.88949 126.06949) (end 177.038 126.218) (width 0.25) (layer B.Cu) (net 1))
 (segment (start 163.83 125.476) (end 163.83 123.972) (width 0.25) (layer B.Cu) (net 9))
 (segment (start 163.83 123.972) (end 164.13027 123.67173) (width 0.25) (layer B.Cu) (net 9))
 (segment (start 164.13027 123.67173) (end 166.023 123.67173) (width 0.25) (layer B.Cu) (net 9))
 (segment (start 163.83 120.576) (end 163.83 122.154) (width 0.25) (layer B.Cu) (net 10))
 (segment (start 163.83 122.154) (end 164.54763 122.87163) (width 0.25) (layer B.Cu) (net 10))
 (segment (start 164.54763 122.87163) (end 166.023 122.87163) (width 0.25) (layer B.Cu) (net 10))
 (segment (start 167.894 116.37559) (end 167.894 116.20159) (width 0.25) (layer B.Cu) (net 11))
 (segment (start 167.894 116.20159) (end 165.688 113.99559) (width 0.25) (layer B.Cu) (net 11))
 (segment (start 165.688 113.99559) (end 163.322 113.99559) (width 0.25) (layer B.Cu) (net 11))
 (segment (start 167.894 116.37559) (end 167.894 116.28159) (width 0.25) (layer B.Cu) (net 11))
 (segment (start 165.989 116.37559) (end 162.734 116.37559) (width 0.25) (layer B.Cu) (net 12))
 (segment (start 161.29 114.93159) (end 161.29 113.99559) (width 0.25) (layer B.Cu) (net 12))
 (segment (start 162.734 116.37559) (end 161.29 114.93159) (width 0.25) (layer B.Cu) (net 12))
 (segment (start 165.989 116.37559) (end 165.989 116.28159) (width 0.25) (layer B.Cu) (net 12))
 (segment (start 159.258 113.99559) (end 159.258 116.12159) (width 0.25) (layer B.Cu) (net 13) (status C00000))
 (segment (start 171.45 114.42359) (end 171.45 115.18559) (width 0.25) (layer B.Cu) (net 2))
 (segment (start 171.45 115.18559) (end 170.18 116.45559) (width 0.25) (layer B.Cu) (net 2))
 (segment (start 170.18 116.45559) (end 170.18 118.48759) (width 0.25) (layer B.Cu) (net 2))
 (segment (start 170.18 118.48759) (end 171.51448 119.82207) (width 0.25) (layer B.Cu) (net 2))
 (segment (start 171.51448 119.82207) (end 171.51448 121.37811) (width 0.25) (layer B.Cu) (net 2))
 (segment (start 174.6082 122.87163) (end 176.53 120.94983) (width 0.25) (layer B.Cu) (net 3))
 (segment (start 176.53 120.94983) (end 176.53 117.47159) (width 0.25) (layer B.Cu) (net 3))
 (segment (start 173.99 114.42359) (end 175.26 113.15359) (width 0.25) (layer B.Cu) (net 3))
 (segment (start 177.8 116.20159) (end 176.53 117.47159) (width 0.25) (layer B.Cu) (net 3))
 (segment (start 177.8 113.91559) (end 177.8 116.20159) (width 0.25) (layer B.Cu) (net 3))
 (segment (start 177.038 113.15359) (end 177.8 113.91559) (width 0.25) (layer B.Cu) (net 3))
 (segment (start 175.26 113.15359) (end 177.038 113.15359) (width 0.25) (layer B.Cu) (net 3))
 (segment (start 173.99 117.47159) (end 173.99 120.50279) (width 0.25) (layer B.Cu) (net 4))
 (segment (start 173.99 120.50279) (end 173.11468 121.37811) (width 0.25) (layer B.Cu) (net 4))
 (segment (start 173.99 117.47159) (end 176.53 114.93159) (width 0.25) (layer B.Cu) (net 4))
 (segment (start 176.53 114.93159) (end 176.53 114.42359) (width 0.25) (layer B.Cu) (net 4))
 (segment (start 169.799 112.89959) (end 169.793498 112.905092) (width 0.25) (layer B.Cu) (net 5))
 (segment (start 175.133 110.48659) (end 170.815 110.48659) (width 0.25) (layer B.Cu) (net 5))
 (segment (start 170.815 110.48659) (end 170.115801 111.185789) (width 0.25) (layer B.Cu) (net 5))
 (segment (start 170.115801 111.185789) (end 170.115801 112.581391) (width 0.25) (layer B.Cu) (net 5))
 (segment (start 170.115801 112.581391) (end 169.799 112.898192) (width 0.25) (layer B.Cu) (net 5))
 (segment (start 169.799 112.898192) (end 169.799 112.89959) (width 0.25) (layer B.Cu) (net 5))
 (segment (start 176.53 111.88359) (end 175.133 110.48659) (width 0.25) (layer B.Cu) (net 5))
 (segment (start 169.91682 119.497206) (end 169.91682 121.37811) (width 0.25) (layer B.Cu) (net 5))
 (segment (start 169.279996 118.860382) (end 169.91682 119.497206) (width 0.25) (layer B.Cu) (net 5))
 (segment (start 169.279996 116.082798) (end 169.279996 118.860382) (width 0.25) (layer B.Cu) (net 5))
 (segment (start 169.793498 115.569296) (end 169.279996 116.082798) (width 0.25) (layer B.Cu) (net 5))
 (segment (start 169.793498 112.905092) (end 169.793498 115.569296) (width 0.25) (layer B.Cu) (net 5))
 (segment (start 172.31458 121.37811) (end 172.31458 118.33617) (width 0.25) (layer B.Cu) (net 6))
 (segment (start 172.31458 118.33617) (end 171.45 117.47159) (width 0.25) (layer B.Cu) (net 6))
 (segment (start 173.99 111.88359) (end 172.72 113.15359) (width 0.25) (layer B.Cu) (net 6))
 (segment (start 172.72 116.20159) (end 171.45 117.47159) (width 0.25) (layer B.Cu) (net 6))
 (segment (start 172.72 113.15359) (end 172.72 116.20159) (width 0.25) (layer B.Cu) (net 6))
 (segment (start 170.71438 121.37811) (end 170.71438 119.658368) (width 0.25) (layer B.Cu) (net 7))
 (segment (start 170.2435 113.09009) (end 171.45 111.88359) (width 0.25) (layer B.Cu) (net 7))
 (segment (start 170.2435 115.755692) (end 170.2435 113.09009) (width 0.25) (layer B.Cu) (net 7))
 (segment (start 169.729998 116.269194) (end 170.2435 115.755692) (width 0.25) (layer B.Cu) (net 7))
 (segment (start 169.729998 118.673986) (end 169.729998 116.269194) (width 0.25) (layer B.Cu) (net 7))
 (segment (start 170.71438 119.658368) (end 169.729998 118.673986) (width 0.25) (layer B.Cu) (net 7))
 (segment (start 167.51652 121.37811) (end 165.95852 121.37811) (width 0.25) (layer B.Cu) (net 16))
 (segment (start 163.402 118.82159) (end 159.258 118.82159) (width 0.25) (layer B.Cu) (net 16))
 (segment (start 165.95852 121.37811) (end 163.402 118.82159) (width 0.25) (layer B.Cu) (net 16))
 (segment (start 167.51652 121.37811) (end 167.51652 121.11452) (width 0.25) (layer B.Cu) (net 16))
 (segment (start 168.31662 121.37811) (end 168.31662 120.56121) (width 0.25) (layer B.Cu) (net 17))
 (segment (start 167.179 120.26559) (end 165.989 119.07559) (width 0.25) (layer B.Cu) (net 17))
 (segment (start 168.021 120.26559) (end 167.179 120.26559) (width 0.25) (layer B.Cu) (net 17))
 (segment (start 168.31662 120.56121) (end 168.021 120.26559) (width 0.25) (layer B.Cu) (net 17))
 (segment (start 169.11672 121.37811) (end 169.11672 120.29831) (width 0.25) (layer B.Cu) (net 18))
 (segment (start 169.11672 120.29831) (end 167.894 119.07559) (width 0.25) (layer B.Cu) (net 18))
 (segment (start 179.959 126.36159) (end 176.35728 129.96331) (width 0.25) (layer B.Cu) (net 24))
 (segment (start 176.35728 129.96331) (end 173.11468 129.96331) (width 0.25) (layer B.Cu) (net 24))
 (segment (start 175.26 131.06059) (end 177.8 131.06059) (width 0.25) (layer B.Cu) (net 25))
 (segment (start 172.31458 130.78217) (end 172.593 131.06059) (width 0.25) (layer B.Cu) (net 25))
 (segment (start 172.593 131.06059) (end 175.26 131.06059) (width 0.25) (layer B.Cu) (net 25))
 (segment (start 172.31458 129.96331) (end 172.31458 130.78217) (width 0.25) (layer B.Cu) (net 25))
 (segment (start 177.8 131.06059) (end 179.959 128.90159) (width 0.25) (layer B.Cu) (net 25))
 (segment (start 171.51448 129.96331) (end 171.51448 130.74407) (width 0.25) (layer B.Cu) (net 26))
 (segment (start 172.281002 131.510592) (end 179.889998 131.510592) (width 0.25) (layer B.Cu) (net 26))
 (segment (start 171.51448 130.74407) (end 172.281002 131.510592) (width 0.25) (layer B.Cu) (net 26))
 (segment (start 179.889998 131.510592) (end 179.959 131.44159) (width 0.25) (layer B.Cu) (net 26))
 (segment (start 170.71438 129.96331) (end 170.71438 130.70597) (width 0.25) (layer B.Cu) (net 27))
 (segment (start 177.938004 131.960594) (end 179.959 133.98159) (width 0.25) (layer B.Cu) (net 27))
 (segment (start 171.969004 131.960594) (end 177.938004 131.960594) (width 0.25) (layer B.Cu) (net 27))
 (segment (start 170.71438 130.70597) (end 171.969004 131.960594) (width 0.25) (layer B.Cu) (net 27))
 (segment (start 169.91682 129.96331) (end 169.91682 131.30541) (width 0.25) (layer B.Cu) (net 28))
 (segment (start 169.91682 131.30541) (end 172.593 133.98159) (width 0.25) (layer B.Cu) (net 28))
 (segment (start 168.5925 131.50509) (end 168.586998 131.510592) (width 0.25) (layer B.Cu) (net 29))
 (segment (start 168.586998 131.510592) (end 166.182206 131.510592) (width 0.25) (layer B.Cu) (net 29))
 (segment (start 165.351204 130.67959) (end 158.877 130.67959) (width 0.25) (layer B.Cu) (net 29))
 (segment (start 166.182206 131.510592) (end 165.351204 130.67959) (width 0.25) (layer B.Cu) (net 29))
 (segment (start 169.11672 129.96331) (end 169.11672 130.98087) (width 0.25) (layer B.Cu) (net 29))
 (segment (start 169.11672 130.98087) (end 168.5925 131.50509) (width 0.25) (layer B.Cu) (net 29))
 (segment (start 168.021 131.06059) (end 166.368602 131.06059) (width 0.25) (layer B.Cu) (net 30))
 (segment (start 168.31662 130.76497) (end 168.021 131.06059) (width 0.25) (layer B.Cu) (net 30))
 (segment (start 168.31662 129.96331) (end 168.31662 130.76497) (width 0.25) (layer B.Cu) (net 30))
 (segment (start 163.447602 128.13959) (end 158.877 128.13959) (width 0.25) (layer B.Cu) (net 30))
 (segment (start 166.368602 131.06059) (end 163.447602 128.13959) (width 0.25) (layer B.Cu) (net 30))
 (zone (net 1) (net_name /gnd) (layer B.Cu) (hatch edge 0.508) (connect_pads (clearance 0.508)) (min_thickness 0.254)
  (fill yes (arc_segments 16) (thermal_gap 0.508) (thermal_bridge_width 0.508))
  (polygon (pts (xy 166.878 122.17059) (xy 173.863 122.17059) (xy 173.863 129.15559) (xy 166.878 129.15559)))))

